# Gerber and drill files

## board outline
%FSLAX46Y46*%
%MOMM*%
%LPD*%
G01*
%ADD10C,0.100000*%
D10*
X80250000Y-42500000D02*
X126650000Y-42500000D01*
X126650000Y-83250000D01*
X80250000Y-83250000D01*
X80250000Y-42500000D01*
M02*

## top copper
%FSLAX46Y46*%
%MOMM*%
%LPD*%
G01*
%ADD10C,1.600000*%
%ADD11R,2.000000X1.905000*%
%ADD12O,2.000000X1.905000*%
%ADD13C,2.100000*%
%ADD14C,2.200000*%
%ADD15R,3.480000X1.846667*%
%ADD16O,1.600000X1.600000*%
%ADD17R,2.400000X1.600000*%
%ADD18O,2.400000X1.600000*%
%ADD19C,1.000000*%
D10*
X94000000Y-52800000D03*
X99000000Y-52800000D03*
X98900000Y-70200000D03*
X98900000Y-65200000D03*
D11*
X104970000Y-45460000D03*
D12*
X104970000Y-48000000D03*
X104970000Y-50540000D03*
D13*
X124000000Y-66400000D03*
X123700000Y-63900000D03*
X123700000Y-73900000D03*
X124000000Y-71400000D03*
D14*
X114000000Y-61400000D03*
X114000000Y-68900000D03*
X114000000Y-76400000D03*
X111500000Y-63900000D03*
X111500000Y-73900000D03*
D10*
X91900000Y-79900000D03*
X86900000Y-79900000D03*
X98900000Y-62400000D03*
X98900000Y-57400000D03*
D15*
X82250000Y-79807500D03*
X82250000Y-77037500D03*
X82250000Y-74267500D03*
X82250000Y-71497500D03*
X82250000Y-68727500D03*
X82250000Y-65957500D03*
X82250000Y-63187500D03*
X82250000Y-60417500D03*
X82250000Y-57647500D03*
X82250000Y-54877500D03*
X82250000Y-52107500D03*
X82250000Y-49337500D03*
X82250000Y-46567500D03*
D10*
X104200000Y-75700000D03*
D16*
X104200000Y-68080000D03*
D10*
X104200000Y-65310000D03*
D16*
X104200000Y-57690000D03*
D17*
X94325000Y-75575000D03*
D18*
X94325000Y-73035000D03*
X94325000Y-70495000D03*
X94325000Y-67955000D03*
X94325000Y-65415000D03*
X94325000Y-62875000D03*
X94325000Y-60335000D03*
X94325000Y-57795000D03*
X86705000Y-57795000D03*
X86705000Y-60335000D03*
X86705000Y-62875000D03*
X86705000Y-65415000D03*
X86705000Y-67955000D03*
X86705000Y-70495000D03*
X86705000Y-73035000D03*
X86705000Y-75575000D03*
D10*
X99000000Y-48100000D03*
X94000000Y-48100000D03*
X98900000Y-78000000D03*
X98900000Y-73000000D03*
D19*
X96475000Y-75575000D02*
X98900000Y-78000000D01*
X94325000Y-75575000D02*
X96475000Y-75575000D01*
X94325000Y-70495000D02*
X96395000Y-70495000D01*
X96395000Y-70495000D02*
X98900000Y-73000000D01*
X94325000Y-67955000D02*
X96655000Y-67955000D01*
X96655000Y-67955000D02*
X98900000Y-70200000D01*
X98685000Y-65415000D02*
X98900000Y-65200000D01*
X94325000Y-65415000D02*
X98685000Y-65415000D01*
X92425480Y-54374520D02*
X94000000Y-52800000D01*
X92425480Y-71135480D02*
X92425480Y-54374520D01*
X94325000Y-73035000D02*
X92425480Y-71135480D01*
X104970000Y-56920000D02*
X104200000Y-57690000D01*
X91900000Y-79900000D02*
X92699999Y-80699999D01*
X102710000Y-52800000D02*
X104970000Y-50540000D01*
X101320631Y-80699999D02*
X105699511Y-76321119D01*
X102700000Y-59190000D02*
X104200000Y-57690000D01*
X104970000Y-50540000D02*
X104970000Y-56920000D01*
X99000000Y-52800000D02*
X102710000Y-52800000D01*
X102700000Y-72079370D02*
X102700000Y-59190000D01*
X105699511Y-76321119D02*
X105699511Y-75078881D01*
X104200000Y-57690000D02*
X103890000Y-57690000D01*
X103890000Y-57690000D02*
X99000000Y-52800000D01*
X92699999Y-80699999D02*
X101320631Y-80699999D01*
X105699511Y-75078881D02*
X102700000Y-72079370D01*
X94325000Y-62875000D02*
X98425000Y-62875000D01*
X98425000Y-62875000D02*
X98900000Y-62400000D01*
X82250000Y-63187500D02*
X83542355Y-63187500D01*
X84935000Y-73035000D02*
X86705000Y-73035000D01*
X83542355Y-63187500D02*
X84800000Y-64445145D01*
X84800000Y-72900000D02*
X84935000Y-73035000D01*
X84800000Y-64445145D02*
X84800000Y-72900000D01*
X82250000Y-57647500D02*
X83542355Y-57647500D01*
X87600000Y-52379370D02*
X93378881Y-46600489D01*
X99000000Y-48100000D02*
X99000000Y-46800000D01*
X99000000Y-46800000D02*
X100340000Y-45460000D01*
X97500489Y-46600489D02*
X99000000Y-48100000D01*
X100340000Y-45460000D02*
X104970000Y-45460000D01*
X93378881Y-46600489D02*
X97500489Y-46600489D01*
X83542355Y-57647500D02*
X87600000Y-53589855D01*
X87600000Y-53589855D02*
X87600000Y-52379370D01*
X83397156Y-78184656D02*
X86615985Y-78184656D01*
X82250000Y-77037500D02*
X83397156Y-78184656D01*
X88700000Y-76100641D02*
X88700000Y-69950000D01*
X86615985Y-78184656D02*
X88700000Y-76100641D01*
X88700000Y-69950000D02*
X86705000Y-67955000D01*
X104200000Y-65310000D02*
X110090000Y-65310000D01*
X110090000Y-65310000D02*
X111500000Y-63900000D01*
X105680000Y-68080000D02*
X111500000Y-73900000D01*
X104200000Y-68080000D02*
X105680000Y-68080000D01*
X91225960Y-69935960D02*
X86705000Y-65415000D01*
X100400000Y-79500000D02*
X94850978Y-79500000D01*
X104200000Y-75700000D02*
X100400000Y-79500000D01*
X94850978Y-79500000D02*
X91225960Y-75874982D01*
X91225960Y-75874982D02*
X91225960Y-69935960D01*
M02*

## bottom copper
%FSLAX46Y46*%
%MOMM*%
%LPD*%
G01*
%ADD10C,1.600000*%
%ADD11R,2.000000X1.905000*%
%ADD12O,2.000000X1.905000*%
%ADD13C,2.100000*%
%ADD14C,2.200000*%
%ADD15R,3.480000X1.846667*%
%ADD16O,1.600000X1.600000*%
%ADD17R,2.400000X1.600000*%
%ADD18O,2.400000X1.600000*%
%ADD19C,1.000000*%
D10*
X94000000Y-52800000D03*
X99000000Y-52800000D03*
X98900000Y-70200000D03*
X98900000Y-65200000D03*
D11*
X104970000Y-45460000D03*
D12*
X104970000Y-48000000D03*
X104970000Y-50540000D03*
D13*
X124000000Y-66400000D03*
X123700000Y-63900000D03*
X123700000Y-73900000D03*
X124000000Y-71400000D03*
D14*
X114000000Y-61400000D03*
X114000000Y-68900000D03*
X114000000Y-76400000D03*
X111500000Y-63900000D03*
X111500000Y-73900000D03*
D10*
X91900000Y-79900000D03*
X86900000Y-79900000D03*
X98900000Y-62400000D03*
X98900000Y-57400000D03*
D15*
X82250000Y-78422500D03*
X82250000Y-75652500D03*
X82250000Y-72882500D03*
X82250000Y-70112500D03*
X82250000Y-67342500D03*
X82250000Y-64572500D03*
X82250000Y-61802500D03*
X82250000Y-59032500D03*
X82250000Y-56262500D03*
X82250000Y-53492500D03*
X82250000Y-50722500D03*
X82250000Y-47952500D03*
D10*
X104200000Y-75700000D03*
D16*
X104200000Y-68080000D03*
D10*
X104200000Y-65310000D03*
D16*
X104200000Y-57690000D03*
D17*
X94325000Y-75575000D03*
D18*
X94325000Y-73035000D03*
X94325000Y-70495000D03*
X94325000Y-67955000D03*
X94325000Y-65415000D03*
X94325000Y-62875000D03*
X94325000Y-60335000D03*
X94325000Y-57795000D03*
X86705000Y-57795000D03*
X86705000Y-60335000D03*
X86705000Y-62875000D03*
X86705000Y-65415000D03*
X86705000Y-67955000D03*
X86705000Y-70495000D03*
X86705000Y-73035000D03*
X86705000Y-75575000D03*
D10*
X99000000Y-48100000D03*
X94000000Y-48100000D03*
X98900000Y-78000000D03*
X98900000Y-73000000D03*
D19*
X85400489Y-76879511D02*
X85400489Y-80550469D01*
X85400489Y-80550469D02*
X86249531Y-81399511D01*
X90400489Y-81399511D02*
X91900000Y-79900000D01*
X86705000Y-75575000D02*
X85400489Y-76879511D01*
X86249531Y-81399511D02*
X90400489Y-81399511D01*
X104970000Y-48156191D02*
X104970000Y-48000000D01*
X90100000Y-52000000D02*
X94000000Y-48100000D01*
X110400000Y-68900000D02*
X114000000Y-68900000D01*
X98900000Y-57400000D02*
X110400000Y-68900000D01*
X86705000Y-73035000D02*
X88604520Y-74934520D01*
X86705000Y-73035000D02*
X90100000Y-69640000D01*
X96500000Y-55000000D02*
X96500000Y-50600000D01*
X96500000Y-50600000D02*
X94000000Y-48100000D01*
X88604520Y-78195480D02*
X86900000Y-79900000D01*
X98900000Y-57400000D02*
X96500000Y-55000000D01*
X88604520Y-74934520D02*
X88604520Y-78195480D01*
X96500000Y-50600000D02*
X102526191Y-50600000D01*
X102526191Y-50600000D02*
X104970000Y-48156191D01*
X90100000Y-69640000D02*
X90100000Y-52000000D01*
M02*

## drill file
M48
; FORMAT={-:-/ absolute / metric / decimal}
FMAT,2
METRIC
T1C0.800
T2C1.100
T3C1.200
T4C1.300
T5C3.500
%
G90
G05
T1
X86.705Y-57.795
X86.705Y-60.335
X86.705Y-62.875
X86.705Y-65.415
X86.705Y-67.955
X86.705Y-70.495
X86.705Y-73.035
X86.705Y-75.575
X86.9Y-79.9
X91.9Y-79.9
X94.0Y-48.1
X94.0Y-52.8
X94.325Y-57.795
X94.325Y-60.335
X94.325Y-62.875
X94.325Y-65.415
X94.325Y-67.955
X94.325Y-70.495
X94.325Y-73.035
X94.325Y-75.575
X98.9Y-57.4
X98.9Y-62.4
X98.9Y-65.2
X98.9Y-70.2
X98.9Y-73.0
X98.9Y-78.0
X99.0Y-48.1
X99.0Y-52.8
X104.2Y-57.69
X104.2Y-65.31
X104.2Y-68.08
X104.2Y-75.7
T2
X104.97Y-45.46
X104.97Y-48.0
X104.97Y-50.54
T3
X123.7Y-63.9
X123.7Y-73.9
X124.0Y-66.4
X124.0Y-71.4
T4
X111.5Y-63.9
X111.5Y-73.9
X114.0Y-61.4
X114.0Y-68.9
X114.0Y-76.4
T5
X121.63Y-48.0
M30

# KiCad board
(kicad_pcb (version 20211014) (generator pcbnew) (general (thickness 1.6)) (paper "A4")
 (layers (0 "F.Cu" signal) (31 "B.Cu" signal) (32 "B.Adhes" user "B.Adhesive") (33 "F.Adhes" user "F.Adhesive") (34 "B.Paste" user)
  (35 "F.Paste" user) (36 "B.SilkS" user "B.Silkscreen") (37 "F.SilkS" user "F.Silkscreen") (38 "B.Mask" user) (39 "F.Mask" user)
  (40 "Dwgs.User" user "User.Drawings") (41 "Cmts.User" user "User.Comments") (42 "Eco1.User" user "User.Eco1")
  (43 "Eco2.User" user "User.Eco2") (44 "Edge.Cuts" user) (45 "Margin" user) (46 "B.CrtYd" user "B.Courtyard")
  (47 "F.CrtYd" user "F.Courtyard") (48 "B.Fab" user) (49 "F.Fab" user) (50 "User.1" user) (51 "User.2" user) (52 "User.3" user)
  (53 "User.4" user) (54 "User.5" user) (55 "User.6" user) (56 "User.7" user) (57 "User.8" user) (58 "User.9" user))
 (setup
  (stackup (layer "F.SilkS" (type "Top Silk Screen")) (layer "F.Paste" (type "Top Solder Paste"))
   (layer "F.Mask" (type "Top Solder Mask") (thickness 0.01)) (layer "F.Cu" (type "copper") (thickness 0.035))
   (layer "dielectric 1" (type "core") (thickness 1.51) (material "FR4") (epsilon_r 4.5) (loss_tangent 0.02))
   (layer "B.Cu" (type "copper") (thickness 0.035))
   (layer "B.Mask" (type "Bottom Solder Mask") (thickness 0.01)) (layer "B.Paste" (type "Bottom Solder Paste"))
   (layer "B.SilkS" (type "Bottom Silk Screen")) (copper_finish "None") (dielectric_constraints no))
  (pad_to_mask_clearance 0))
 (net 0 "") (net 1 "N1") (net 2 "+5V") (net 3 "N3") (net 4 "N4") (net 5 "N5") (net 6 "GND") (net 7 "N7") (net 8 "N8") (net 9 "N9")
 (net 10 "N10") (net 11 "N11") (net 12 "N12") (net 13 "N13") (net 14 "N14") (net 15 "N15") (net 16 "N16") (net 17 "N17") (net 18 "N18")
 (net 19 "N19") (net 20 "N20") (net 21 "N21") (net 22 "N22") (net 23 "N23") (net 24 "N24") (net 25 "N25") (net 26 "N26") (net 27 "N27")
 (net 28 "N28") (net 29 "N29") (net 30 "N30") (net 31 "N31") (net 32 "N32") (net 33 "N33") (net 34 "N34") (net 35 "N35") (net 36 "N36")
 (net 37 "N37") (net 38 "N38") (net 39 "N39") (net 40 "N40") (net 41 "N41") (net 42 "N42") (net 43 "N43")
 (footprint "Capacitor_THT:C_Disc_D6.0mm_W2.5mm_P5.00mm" (layer "F.Cu") (at 94 52.8)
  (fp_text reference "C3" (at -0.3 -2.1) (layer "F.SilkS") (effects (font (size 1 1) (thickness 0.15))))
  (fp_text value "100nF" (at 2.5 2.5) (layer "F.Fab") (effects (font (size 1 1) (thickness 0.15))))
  (pad "1" thru_hole circle (at 0 0) (size 1.6 1.6) (drill 0.8) (layers *.Cu *.Mask) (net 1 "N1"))
  (pad "2" thru_hole circle (at 5 0) (size 1.6 1.6) (drill 0.8) (layers *.Cu *.Mask) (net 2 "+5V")))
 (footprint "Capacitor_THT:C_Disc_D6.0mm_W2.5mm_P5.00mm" (layer "F.Cu") (at 98.9 70.2 90)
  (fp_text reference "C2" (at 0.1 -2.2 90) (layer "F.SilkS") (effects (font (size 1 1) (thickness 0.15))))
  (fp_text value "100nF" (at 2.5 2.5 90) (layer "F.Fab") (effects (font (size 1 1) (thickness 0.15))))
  (pad "1" thru_hole circle (at 0 0 90) (size 1.6 1.6) (drill 0.8) (layers *.Cu *.Mask) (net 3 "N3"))
  (pad "2" thru_hole circle (at 5 0 90) (size 1.6 1.6) (drill 0.8) (layers *.Cu *.Mask) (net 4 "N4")))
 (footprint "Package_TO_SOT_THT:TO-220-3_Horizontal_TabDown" (layer "F.Cu") (at 104.97 45.46 -90)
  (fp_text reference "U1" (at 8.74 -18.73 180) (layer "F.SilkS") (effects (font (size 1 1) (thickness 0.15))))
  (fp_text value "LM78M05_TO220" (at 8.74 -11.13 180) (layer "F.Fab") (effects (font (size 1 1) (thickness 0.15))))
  (pad "" np_thru_hole oval (at 2.54 -16.66 270) (size 3.5 3.5) (drill 3.5) (layers *.Cu *.Mask))
  (pad "1" thru_hole rect (at 0 0 270) (size 1.905 2) (drill 1.1) (layers *.Cu *.Mask) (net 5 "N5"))
  (pad "2" thru_hole oval (at 2.54 0 270) (size 1.905 2) (drill 1.1) (layers *.Cu *.Mask) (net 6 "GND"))
  (pad "3" thru_hole oval (at 5.08 0 270) (size 1.905 2) (drill 1.1) (layers *.Cu *.Mask) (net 2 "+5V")))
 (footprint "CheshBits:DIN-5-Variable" (layer "F.Cu") (at 114 68.9 -90)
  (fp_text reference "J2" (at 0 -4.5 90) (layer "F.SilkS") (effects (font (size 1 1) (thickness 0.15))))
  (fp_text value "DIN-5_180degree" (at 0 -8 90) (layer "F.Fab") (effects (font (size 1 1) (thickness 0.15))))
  (pad "" thru_hole circle (at -2.5 -10 270) (size 2.1 2.1) (drill 1.2) (layers *.Cu *.Mask))
  (pad "" thru_hole circle (at -5 -9.7 270) (size 2.1 2.1) (drill 1.2) (layers *.Cu *.Mask))
  (pad "" thru_hole circle (at 5 -9.7 270) (size 2.1 2.1) (drill 1.2) (layers *.Cu *.Mask))
  (pad "" thru_hole circle (at 2.5 -10 270) (size 2.1 2.1) (drill 1.2) (layers *.Cu *.Mask))
  (pad "1" thru_hole circle (at -7.5 0 270) (size 2.2 2.2) (drill 1.3) (layers *.Cu *.Mask) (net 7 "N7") (solder_mask_margin 0.15)
   (clearance 0.3))
  (pad "2" thru_hole circle (at 0 0 270) (size 2.2 2.2) (drill 1.3) (layers *.Cu *.Mask) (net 6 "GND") (solder_mask_margin 0.15)
   (clearance 0.3))
  (pad "3" thru_hole circle (at 7.5 0 270) (size 2.2 2.2) (drill 1.3) (layers *.Cu *.Mask) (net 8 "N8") (solder_mask_margin 0.15)
   (clearance 0.3))
  (pad "4" thru_hole circle (at -5 2.5 270) (size 2.2 2.2) (drill 1.3) (layers *.Cu *.Mask) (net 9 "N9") (solder_mask_margin 0.15)
   (clearance 0.3))
  (pad "5" thru_hole circle (at 5 2.5 270) (size 2.2 2.2) (drill 1.3) (layers *.Cu *.Mask) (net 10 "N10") (solder_mask_margin 0.15)
   (clearance 0.3)))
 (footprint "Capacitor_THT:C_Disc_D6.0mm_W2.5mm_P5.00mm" (layer "F.Cu") (at 91.9 79.9 180)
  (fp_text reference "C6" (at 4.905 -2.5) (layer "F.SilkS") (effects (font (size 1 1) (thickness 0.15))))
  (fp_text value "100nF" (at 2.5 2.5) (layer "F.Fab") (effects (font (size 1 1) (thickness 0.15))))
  (pad "1" thru_hole circle (at 0 0 180) (size 1.6 1.6) (drill 0.8) (layers *.Cu *.Mask) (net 2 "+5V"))
  (pad "2" thru_hole circle (at 5 0 180) (size 1.6 1.6) (drill 0.8) (layers *.Cu *.Mask) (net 6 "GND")))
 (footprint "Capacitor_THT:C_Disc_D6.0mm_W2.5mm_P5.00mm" (layer "F.Cu") (at 98.9 62.4 90)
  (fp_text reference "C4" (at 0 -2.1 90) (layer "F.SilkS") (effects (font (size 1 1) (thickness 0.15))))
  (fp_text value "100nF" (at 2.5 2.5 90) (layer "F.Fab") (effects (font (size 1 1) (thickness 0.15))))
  (pad "1" thru_hole circle (at 0 0 90) (size 1.6 1.6) (drill 0.8) (layers *.Cu *.Mask) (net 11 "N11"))
  (pad "2" thru_hole circle (at 5 0 90) (size 1.6 1.6) (drill 0.8) (layers *.Cu *.Mask) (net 6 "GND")))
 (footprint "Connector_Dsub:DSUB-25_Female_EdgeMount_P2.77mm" (layer "F.Cu") (at 82.25 63.1875 -90)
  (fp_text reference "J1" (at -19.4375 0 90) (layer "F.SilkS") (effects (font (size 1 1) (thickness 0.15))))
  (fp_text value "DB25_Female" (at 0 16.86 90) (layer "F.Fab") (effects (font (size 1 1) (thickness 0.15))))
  (pad "1" smd rect (at 16.62 0 270) (size 1.846667 3.48) (layers "F.Cu" "F.Paste" "F.Mask") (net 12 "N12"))
  (pad "2" smd rect (at 13.85 0 270) (size 1.846667 3.48) (layers "F.Cu" "F.Paste" "F.Mask") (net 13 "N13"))
  (pad "3" smd rect (at 11.08 0 270) (size 1.846667 3.48) (layers "F.Cu" "F.Paste" "F.Mask") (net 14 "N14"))
  (pad "4" smd rect (at 8.31 0 270) (size 1.846667 3.48) (layers "F.Cu" "F.Paste" "F.Mask") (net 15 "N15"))
  (pad "5" smd rect (at 5.54 0 270) (size 1.846667 3.48) (layers "F.Cu" "F.Paste" "F.Mask") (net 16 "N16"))
  (pad "6" smd rect (at 2.77 0 270) (size 1.846667 3.48) (layers "F.Cu" "F.Paste" "F.Mask") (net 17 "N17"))
  (pad "7" smd rect (at 0 0 270) (size 1.846667 3.48) (layers "F.Cu" "F.Paste" "F.Mask") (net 6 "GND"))
  (pad "8" smd rect (at -2.77 0 270) (size 1.846667 3.48) (layers "F.Cu" "F.Paste" "F.Mask") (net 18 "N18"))
  (pad "9" smd rect (at -5.54 0 270) (size 1.846667 3.48) (layers "F.Cu" "F.Paste" "F.Mask") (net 5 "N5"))
  (pad "10" smd rect (at -8.31 0 270) (size 1.846667 3.48) (layers "F.Cu" "F.Paste" "F.Mask") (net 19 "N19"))
  (pad "11" smd rect (at -11.08 0 270) (size 1.846667 3.48) (layers "F.Cu" "F.Paste" "F.Mask") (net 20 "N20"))
  (pad "12" smd rect (at -13.85 0 270) (size 1.846667 3.48) (layers "F.Cu" "F.Paste" "F.Mask") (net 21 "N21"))
  (pad "13" smd rect (at -16.62 0 270) (size 1.846667 3.48) (layers "F.Cu" "F.Paste" "F.Mask") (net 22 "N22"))
  (pad "14" smd rect (at 15.235 0 270) (size 1.846667 3.48) (layers "B.Cu" "B.Paste" "B.Mask") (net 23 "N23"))
  (pad "15" smd rect (at 12.465 0 270) (size 1.846667 3.48) (layers "B.Cu" "B.Paste" "B.Mask") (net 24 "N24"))
  (pad "16" smd rect (at 9.695 0 270) (size 1.846667 3.48) (layers "B.Cu" "B.Paste" "B.Mask") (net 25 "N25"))
  (pad "17" smd rect (at 6.925 0 270) (size 1.846667 3.48) (layers "B.Cu" "B.Paste" "B.Mask") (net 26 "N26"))
  (pad "18" smd rect (at 4.155 0 270) (size 1.846667 3.48) (layers "B.Cu" "B.Paste" "B.Mask") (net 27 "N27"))
  (pad "19" smd rect (at 1.385 0 270) (size 1.846667 3.48) (layers "B.Cu" "B.Paste" "B.Mask") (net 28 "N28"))
  (pad "20" smd rect (at -1.385 0 270) (size 1.846667 3.48) (layers "B.Cu" "B.Paste" "B.Mask") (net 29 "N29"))
  (pad "21" smd rect (at -4.155 0 270) (size 1.846667 3.48) (layers "B.Cu" "B.Paste" "B.Mask") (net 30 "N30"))
  (pad "22" smd rect (at -6.925 0 270) (size 1.846667 3.48) (layers "B.Cu" "B.Paste" "B.Mask") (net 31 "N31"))
  (pad "23" smd rect (at -9.695 0 270) (size 1.846667 3.48) (layers "B.Cu" "B.Paste" "B.Mask") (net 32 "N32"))
  (pad "24" smd rect (at -12.465 0 270) (size 1.846667 3.48) (layers "B.Cu" "B.Paste" "B.Mask") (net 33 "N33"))
  (pad "25" smd rect (at -15.235 0 270) (size 1.846667 3.48) (layers "B.Cu" "B.Paste" "B.Mask") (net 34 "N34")))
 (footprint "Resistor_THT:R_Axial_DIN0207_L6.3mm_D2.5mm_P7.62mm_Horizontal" (layer "F.Cu") (at 104.2 75.7 90)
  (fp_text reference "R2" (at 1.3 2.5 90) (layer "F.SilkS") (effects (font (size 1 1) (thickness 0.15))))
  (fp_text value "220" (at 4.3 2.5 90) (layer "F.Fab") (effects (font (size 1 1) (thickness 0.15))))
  (pad "1" thru_hole circle (at 0 0 90) (size 1.6 1.6) (drill 0.8) (layers *.Cu *.Mask) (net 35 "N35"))
  (pad "2" thru_hole oval (at 7.62 0 90) (size 1.6 1.6) (drill 0.8) (layers *.Cu *.Mask) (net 10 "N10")))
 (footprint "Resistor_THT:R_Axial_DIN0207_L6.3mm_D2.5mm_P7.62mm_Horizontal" (layer "F.Cu") (at 104.2 65.31 90)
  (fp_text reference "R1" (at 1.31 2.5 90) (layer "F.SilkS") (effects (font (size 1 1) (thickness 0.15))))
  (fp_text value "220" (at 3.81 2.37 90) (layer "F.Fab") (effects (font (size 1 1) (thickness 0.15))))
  (pad "1" thru_hole circle (at 0 0 90) (size 1.6 1.6) (drill 0.8) (layers *.Cu *.Mask) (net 9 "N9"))
  (pad "2" thru_hole oval (at 7.62 0 90) (size 1.6 1.6) (drill 0.8) (layers *.Cu *.Mask) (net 2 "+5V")))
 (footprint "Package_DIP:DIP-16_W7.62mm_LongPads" (layer "F.Cu") (at 94.325 75.575 180)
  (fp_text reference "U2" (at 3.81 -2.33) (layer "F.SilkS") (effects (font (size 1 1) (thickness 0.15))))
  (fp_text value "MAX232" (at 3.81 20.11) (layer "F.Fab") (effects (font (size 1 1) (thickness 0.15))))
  (pad "1" thru_hole rect (at 0 0 180) (size 2.4 1.6) (drill 0.8) (layers *.Cu *.Mask) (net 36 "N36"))
  (pad "2" thru_hole oval (at 0 2.54 180) (size 2.4 1.6) (drill 0.8) (layers *.Cu *.Mask) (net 1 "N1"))
  (pad "3" thru_hole oval (at 0 5.08 180) (size 2.4 1.6) (drill 0.8) (layers *.Cu *.Mask) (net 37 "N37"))
  (pad "4" thru_hole oval (at 0 7.62 180) (size 2.4 1.6) (drill 0.8) (layers *.Cu *.Mask) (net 3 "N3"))
  (pad "5" thru_hole oval (at 0 10.16 180) (size 2.4 1.6) (drill 0.8) (layers *.Cu *.Mask) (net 4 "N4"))
  (pad "6" thru_hole oval (at 0 12.7 180) (size 2.4 1.6) (drill 0.8) (layers *.Cu *.Mask) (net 11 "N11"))
  (pad "7" thru_hole oval (at 0 15.24 180) (size 2.4 1.6) (drill 0.8) (layers *.Cu *.Mask) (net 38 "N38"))
  (pad "8" thru_hole oval (at 0 17.78 180) (size 2.4 1.6) (drill 0.8) (layers *.Cu *.Mask) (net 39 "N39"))
  (pad "9" thru_hole oval (at 7.62 17.78 180) (size 2.4 1.6) (drill 0.8) (layers *.Cu *.Mask) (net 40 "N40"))
  (pad "10" thru_hole oval (at 7.62 15.24 180) (size 2.4 1.6) (drill 0.8) (layers *.Cu *.Mask) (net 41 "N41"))
  (pad "11" thru_hole oval (at 7.62 12.7 180) (size 2.4 1.6) (drill 0.8) (layers *.Cu *.Mask) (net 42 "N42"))
  (pad "12" thru_hole oval (at 7.62 10.16 180) (size 2.4 1.6) (drill 0.8) (layers *.Cu *.Mask) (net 35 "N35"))
  (pad "13" thru_hole oval (at 7.62 7.62 180) (size 2.4 1.6) (drill 0.8) (layers *.Cu *.Mask) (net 13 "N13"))
  (pad "14" thru_hole oval (at 7.62 5.08 180) (size 2.4 1.6) (drill 0.8) (layers *.Cu *.Mask) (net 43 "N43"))
  (pad "15" thru_hole oval (at 7.62 2.54 180) (size 2.4 1.6) (drill 0.8) (layers *.Cu *.Mask) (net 6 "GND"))
  (pad "16" thru_hole oval (at 7.62 0 180) (size 2.4 1.6) (drill 0.8) (layers *.Cu *.Mask) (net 2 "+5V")))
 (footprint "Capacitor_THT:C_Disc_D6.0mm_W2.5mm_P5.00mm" (layer "F.Cu") (at 99 48.1 180)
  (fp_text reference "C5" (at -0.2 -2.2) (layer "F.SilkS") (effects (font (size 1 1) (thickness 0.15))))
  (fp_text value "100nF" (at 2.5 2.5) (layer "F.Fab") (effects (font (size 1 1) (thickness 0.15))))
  (pad "1" thru_hole circle (at 0 0 180) (size 1.6 1.6) (drill 0.8) (layers *.Cu *.Mask) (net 5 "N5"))
  (pad "2" thru_hole circle (at 5 0 180) (size 1.6 1.6) (drill 0.8) (layers *.Cu *.Mask) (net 6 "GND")))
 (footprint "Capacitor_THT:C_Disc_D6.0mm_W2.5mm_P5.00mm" (layer "F.Cu") (at 98.9 78 90)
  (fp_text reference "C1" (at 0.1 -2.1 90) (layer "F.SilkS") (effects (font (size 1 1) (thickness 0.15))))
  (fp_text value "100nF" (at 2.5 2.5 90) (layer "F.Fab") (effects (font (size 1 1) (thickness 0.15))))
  (pad "1" thru_hole circle (at 0 0 90) (size 1.6 1.6) (drill 0.8) (layers *.Cu *.Mask) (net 36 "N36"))
  (pad "2" thru_hole circle (at 5 0 90) (size 1.6 1.6) (drill 0.8) (layers *.Cu *.Mask) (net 37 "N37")))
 (gr_rect (start 80.25 42.5) (end 126.65 83.25) (layer "Edge.Cuts") (width 0.1) (fill none))
 (segment (start 96.475 75.575) (end 98.9 78) (width 1) (layer "F.Cu") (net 36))
 (segment (start 94.325 75.575) (end 96.475 75.575) (width 1) (layer "F.Cu") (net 36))
 (segment (start 94.325 70.495) (end 96.395 70.495) (width 1) (layer "F.Cu") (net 37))
 (segment (start 96.395 70.495) (end 98.9 73) (width 1) (layer "F.Cu") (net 37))
 (segment (start 94.325 67.955) (end 96.655 67.955) (width 1) (layer "F.Cu") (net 3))
 (segment (start 96.655 67.955) (end 98.9 70.2) (width 1) (layer "F.Cu") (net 3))
 (segment (start 98.685 65.415) (end 98.9 65.2) (width 1) (layer "F.Cu") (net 4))
 (segment (start 94.325 65.415) (end 98.685 65.415) (width 1) (layer "F.Cu") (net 4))
 (segment (start 92.42548 54.37452) (end 94 52.8) (width 1) (layer "F.Cu") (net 1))
 (segment (start 92.42548 71.13548) (end 92.42548 54.37452) (width 1) (layer "F.Cu") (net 1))
 (segment (start 94.325 73.035) (end 92.42548 71.13548) (width 1) (layer "F.Cu") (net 1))
 (segment (start 104.97 56.92) (end 104.2 57.69) (width 1) (layer "F.Cu") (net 2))
 (segment (start 91.9 79.9) (end 92.699999 80.699999) (width 1) (layer "F.Cu") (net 2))
 (segment (start 102.71 52.8) (end 104.97 50.54) (width 1) (layer "F.Cu") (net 2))
 (segment (start 101.320631 80.699999) (end 105.699511 76.321119) (width 1) (layer "F.Cu") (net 2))
 (segment (start 102.7 59.19) (end 104.2 57.69) (width 1) (layer "F.Cu") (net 2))
 (segment (start 104.97 50.54) (end 104.97 56.92) (width 1) (layer "F.Cu") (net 2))
 (segment (start 99 52.8) (end 102.71 52.8) (width 1) (layer "F.Cu") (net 2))
 (segment (start 102.7 72.07937) (end 102.7 59.19) (width 1) (layer "F.Cu") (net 2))
 (segment (start 105.699511 76.321119) (end 105.699511 75.078881) (width 1) (layer "F.Cu") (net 2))
 (segment (start 104.2 57.69) (end 103.89 57.69) (width 1) (layer "F.Cu") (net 2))
 (segment (start 103.89 57.69) (end 99 52.8) (width 1) (layer "F.Cu") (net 2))
 (segment (start 92.699999 80.699999) (end 101.320631 80.699999) (width 1) (layer "F.Cu") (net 2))
 (segment (start 105.699511 75.078881) (end 102.7 72.07937) (width 1) (layer "F.Cu") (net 2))
 (segment (start 85.400489 76.879511) (end 85.400489 80.550469) (width 1) (layer "B.Cu") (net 2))
 (segment (start 85.400489 80.550469) (end 86.249531 81.399511) (width 1) (layer "B.Cu") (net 2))
 (segment (start 90.400489 81.399511) (end 91.9 79.9) (width 1) (layer "B.Cu") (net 2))
 (segment (start 86.705 75.575) (end 85.400489 76.879511) (width 1) (layer "B.Cu") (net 2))
 (segment (start 86.249531 81.399511) (end 90.400489 81.399511) (width 1) (layer "B.Cu") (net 2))
 (segment (start 94.325 62.875) (end 98.425 62.875) (width 1) (layer "F.Cu") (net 11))
 (segment (start 98.425 62.875) (end 98.9 62.4) (width 1) (layer "F.Cu") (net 11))
 (segment (start 82.25 63.1875) (end 83.542355 63.1875) (width 1) (layer "F.Cu") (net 6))
 (segment (start 84.935 73.035) (end 86.705 73.035) (width 1) (layer "F.Cu") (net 6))
 (segment (start 83.542355 63.1875) (end 84.8 64.445145) (width 1) (layer "F.Cu") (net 6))
 (segment (start 84.8 72.9) (end 84.935 73.035) (width 1) (layer "F.Cu") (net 6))
 (segment (start 84.8 64.445145) (end 84.8 72.9) (width 1) (layer "F.Cu") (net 6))
 (segment (start 104.97 48.156191) (end 104.97 48) (width 1) (layer "B.Cu") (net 6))
 (segment (start 90.1 52) (end 94 48.1) (width 1) (layer "B.Cu") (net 6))
 (segment (start 110.4 68.9) (end 114 68.9) (width 1) (layer "B.Cu") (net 6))
 (segment (start 98.9 57.4) (end 110.4 68.9) (width 1) (layer "B.Cu") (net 6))
 (segment (start 86.705 73.035) (end 88.60452 74.93452) (width 1) (layer "B.Cu") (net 6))
 (segment (start 86.705 73.035) (end 90.1 69.64) (width 1) (layer "B.Cu") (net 6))
 (segment (start 96.5 55) (end 96.5 50.6) (width 1) (layer "B.Cu") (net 6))
 (segment (start 96.5 50.6) (end 94 48.1) (width 1) (layer "B.Cu") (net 6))
 (segment (start 88.60452 78.19548) (end 86.9 79.9) (width 1) (layer "B.Cu") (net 6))
 (segment (start 98.9 57.4) (end 96.5 55) (width 1) (layer "B.Cu") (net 6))
 (segment (start 88.60452 74.93452) (end 88.60452 78.19548) (width 1) (layer "B.Cu") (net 6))
 (segment (start 96.5 50.6) (end 102.526191 50.6) (width 1) (layer "B.Cu") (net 6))
 (segment (start 102.526191 50.6) (end 104.97 48.156191) (width 1) (layer "B.Cu") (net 6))
 (segment (start 90.1 69.64) (end 90.1 52) (width 1) (layer "B.Cu") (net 6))
 (segment (start 82.25 57.6475) (end 83.542355 57.6475) (width 1) (layer "F.Cu") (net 5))
 (segment (start 87.6 52.37937) (end 93.378881 46.600489) (width 1) (layer "F.Cu") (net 5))
 (segment (start 99 48.1) (end 99 46.8) (width 1) (layer "F.Cu") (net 5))
 (segment (start 99 46.8) (end 100.34 45.46) (width 1) (layer "F.Cu") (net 5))
 (segment (start 97.500489 46.600489) (end 99 48.1) (width 1) (layer "F.Cu") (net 5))
 (segment (start 100.34 45.46) (end 104.97 45.46) (width 1) (layer "F.Cu") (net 5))
 (segment (start 93.378881 46.600489) (end 97.500489 46.600489) (width 1) (layer "F.Cu") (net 5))
 (segment (start 83.542355 57.6475) (end 87.6 53.589855) (width 1) (layer "F.Cu") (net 5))
 (segment (start 87.6 53.589855) (end 87.6 52.37937) (width 1) (layer "F.Cu") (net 5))
 (segment (start 83.397156 78.184656) (end 86.615985 78.184656) (width 1) (layer "F.Cu") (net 13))
 (segment (start 82.25 77.0375) (end 83.397156 78.184656) (width 1) (layer "F.Cu") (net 13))
 (segment (start 88.7 76.100641) (end 88.7 69.95) (width 1) (layer "F.Cu") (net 13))
 (segment (start 86.615985 78.184656) (end 88.7 76.100641) (width 1) (layer "F.Cu") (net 13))
 (segment (start 88.7 69.95) (end 86.705 67.955) (width 1) (layer "F.Cu") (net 13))
 (segment (start 104.2 65.31) (end 110.09 65.31) (width 1) (layer "F.Cu") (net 9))
 (segment (start 110.09 65.31) (end 111.5 63.9) (width 1) (layer "F.Cu") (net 9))
 (segment (start 105.68 68.08) (end 111.5 73.9) (width 1) (layer "F.Cu") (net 10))
 (segment (start 104.2 68.08) (end 105.68 68.08) (width 1) (layer "F.Cu") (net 10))
 (segment (start 91.22596 69.93596) (end 86.705 65.415) (width 1) (layer "F.Cu") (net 35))
 (segment (start 100.4 79.5) (end 94.850978 79.5) (width 1) (layer "F.Cu") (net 35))
 (segment (start 104.2 75.7) (end 100.4 79.5) (width 1) (layer "F.Cu") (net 35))
 (segment (start 94.850978 79.5) (end 91.22596 75.874982) (width 1) (layer "F.Cu") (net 35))
 (segment (start 91.22596 75.874982) (end 91.22596 69.93596) (width 1) (layer "F.Cu") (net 35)))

